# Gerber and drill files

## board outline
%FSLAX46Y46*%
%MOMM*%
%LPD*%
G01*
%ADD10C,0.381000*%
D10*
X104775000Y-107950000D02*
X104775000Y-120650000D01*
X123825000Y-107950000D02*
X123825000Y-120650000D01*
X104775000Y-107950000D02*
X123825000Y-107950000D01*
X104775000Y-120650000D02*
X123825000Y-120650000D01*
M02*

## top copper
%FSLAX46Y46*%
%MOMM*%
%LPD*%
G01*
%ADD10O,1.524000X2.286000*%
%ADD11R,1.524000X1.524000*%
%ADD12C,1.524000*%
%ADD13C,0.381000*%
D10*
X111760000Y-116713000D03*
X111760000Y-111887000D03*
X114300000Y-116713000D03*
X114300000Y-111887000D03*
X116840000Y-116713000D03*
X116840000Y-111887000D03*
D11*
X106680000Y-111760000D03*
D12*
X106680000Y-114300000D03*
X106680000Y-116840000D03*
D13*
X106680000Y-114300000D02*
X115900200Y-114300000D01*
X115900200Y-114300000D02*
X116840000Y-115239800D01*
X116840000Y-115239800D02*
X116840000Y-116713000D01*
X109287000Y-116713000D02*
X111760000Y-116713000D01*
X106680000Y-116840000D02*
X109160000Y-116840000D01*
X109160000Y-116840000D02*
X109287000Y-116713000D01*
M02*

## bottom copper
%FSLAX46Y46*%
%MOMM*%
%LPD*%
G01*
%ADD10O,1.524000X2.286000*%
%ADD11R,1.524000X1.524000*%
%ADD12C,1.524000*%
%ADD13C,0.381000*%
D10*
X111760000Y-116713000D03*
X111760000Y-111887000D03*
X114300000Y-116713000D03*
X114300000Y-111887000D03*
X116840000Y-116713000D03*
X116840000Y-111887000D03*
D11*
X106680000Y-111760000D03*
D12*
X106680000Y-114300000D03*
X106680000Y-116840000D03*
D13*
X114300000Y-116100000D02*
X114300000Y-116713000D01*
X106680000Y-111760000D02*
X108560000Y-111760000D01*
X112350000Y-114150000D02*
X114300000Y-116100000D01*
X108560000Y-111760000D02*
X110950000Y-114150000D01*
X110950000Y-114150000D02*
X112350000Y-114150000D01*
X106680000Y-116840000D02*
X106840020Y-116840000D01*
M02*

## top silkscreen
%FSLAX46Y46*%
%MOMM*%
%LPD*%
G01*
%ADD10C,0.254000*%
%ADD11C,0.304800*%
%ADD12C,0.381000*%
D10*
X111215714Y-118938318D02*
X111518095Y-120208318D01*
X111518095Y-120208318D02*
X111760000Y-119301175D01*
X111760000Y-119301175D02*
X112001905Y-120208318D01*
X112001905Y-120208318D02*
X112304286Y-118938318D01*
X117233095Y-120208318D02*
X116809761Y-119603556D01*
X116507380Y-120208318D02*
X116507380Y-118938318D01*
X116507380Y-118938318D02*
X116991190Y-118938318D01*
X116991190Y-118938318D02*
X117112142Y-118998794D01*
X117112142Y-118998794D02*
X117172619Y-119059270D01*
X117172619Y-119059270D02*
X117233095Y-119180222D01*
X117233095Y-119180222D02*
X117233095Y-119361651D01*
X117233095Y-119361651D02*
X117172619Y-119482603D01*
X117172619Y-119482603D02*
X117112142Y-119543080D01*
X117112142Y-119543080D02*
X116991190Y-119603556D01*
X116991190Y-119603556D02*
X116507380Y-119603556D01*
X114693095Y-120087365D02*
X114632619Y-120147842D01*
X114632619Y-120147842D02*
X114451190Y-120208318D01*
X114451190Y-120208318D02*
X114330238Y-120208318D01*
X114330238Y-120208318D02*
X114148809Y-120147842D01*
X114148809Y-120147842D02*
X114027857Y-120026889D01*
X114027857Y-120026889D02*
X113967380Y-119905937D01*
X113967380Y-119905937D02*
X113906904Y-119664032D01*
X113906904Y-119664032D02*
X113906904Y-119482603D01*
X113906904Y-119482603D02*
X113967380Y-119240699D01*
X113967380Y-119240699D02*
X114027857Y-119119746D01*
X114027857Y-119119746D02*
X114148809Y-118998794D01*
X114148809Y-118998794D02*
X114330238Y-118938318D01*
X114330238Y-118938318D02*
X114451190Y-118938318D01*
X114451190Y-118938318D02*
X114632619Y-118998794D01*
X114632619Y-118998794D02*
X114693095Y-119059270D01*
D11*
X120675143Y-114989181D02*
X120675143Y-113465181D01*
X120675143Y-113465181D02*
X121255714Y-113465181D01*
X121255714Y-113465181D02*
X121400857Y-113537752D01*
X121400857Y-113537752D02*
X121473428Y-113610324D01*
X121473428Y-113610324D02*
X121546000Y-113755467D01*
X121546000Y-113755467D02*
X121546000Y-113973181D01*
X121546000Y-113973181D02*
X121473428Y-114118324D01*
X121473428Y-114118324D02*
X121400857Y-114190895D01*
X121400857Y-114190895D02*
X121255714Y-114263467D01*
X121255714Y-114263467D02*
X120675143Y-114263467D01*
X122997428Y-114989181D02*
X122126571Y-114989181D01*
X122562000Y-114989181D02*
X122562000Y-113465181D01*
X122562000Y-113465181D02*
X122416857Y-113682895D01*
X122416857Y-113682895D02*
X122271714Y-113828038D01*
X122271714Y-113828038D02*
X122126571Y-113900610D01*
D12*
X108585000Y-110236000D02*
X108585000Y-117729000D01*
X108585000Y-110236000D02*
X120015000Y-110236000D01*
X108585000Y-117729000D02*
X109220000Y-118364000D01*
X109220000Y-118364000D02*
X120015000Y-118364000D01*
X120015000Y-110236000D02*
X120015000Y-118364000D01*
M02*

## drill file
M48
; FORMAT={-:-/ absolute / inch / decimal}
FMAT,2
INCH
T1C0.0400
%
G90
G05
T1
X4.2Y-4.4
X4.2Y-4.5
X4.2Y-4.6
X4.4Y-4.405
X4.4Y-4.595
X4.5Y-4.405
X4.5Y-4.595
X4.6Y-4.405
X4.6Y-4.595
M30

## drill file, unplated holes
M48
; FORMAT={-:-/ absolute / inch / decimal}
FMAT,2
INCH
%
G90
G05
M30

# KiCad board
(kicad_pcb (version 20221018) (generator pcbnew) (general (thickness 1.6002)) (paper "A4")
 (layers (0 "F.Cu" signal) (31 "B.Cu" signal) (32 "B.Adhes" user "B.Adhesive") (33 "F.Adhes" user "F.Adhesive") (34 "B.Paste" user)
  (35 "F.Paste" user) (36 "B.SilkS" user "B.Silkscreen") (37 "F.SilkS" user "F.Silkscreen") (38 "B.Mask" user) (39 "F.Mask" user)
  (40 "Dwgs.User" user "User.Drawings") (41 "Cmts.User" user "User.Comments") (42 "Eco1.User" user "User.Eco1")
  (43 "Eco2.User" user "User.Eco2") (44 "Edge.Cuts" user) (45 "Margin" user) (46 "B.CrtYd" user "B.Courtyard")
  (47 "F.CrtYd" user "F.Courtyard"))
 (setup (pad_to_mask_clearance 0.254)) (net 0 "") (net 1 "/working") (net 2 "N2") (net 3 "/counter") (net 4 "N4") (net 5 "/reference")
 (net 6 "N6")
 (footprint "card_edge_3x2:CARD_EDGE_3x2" (layer "F.Cu") (at 114.3 114.3)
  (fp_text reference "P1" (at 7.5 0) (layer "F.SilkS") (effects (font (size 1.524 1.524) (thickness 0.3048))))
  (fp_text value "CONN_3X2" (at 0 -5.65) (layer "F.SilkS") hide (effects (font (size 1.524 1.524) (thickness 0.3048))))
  (fp_line (start -5.715 -4.064) (end -5.715 3.429) (stroke (width 0.381) (type solid)) (layer "F.SilkS"))
  (fp_line (start -5.715 -4.064) (end 5.715 -4.064) (stroke (width 0.381) (type solid)) (layer "F.SilkS"))
  (fp_line (start -5.715 3.429) (end -5.08 4.064) (stroke (width 0.381) (type solid)) (layer "F.SilkS"))
  (fp_line (start -5.08 4.064) (end 5.715 4.064) (stroke (width 0.381) (type solid)) (layer "F.SilkS"))
  (fp_line (start 5.715 -4.064) (end 5.715 4.064) (stroke (width 0.381) (type solid)) (layer "F.SilkS"))
  (pad "1" thru_hole oval (at -2.54 2.413) (size 1.524 2.286) (drill 1.016) (layers "*.Cu" "*.Mask") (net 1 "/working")
   (thermal_bridge_angle 45))
  (pad "2" thru_hole oval (at -2.54 -2.413) (size 1.524 2.286) (drill 1.016) (layers "*.Cu" "*.Mask") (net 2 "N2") (thermal_bridge_angle 45))
  (pad "3" thru_hole oval (at 0 2.413) (size 1.524 2.286) (drill 1.016) (layers "*.Cu" "*.Mask") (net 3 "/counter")
   (thermal_bridge_angle 45))
  (pad "4" thru_hole oval (at 0 -2.413) (size 1.524 2.286) (drill 1.016) (layers "*.Cu" "*.Mask") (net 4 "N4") (thermal_bridge_angle 45))
  (pad "5" thru_hole oval (at 2.54 2.413) (size 1.524 2.286) (drill 1.016) (layers "*.Cu" "*.Mask") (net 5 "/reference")
   (thermal_bridge_angle 45))
  (pad "6" thru_hole oval (at 2.54 -2.413) (size 1.524 2.286) (drill 1.016) (layers "*.Cu" "*.Mask") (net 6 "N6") (thermal_bridge_angle 45)))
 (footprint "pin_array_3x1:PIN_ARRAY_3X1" (layer "B.Cu") (at 106.68 114.3 -90)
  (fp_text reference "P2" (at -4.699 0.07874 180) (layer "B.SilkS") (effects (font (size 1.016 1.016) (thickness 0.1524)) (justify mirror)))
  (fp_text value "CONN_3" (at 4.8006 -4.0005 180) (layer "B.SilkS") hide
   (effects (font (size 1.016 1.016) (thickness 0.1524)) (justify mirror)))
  (pad "1" thru_hole rect (at -2.54 0 270) (size 1.524 1.524) (drill 1.016) (layers "*.Cu" "*.Mask") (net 3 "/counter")
   (thermal_bridge_angle 45))
  (pad "2" thru_hole circle (at 0 0 270) (size 1.524 1.524) (drill 1.016) (layers "*.Cu" "*.Mask") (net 5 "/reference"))
  (pad "3" thru_hole circle (at 2.54 0 270) (size 1.524 1.524) (drill 1.016) (layers "*.Cu" "*.Mask") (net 1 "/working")))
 (gr_line (start 104.775 107.95) (end 104.775 120.65) (stroke (width 0.381) (type solid)) (layer "Edge.Cuts"))
 (gr_line (start 123.825 107.95) (end 123.825 120.65) (stroke (width 0.381) (type solid)) (layer "Edge.Cuts"))
 (gr_line (start 104.775 107.95) (end 123.825 107.95) (stroke (width 0.381) (type solid)) (layer "Edge.Cuts"))
 (gr_line (start 104.775 120.65) (end 123.825 120.65) (stroke (width 0.381) (type solid)) (layer "Edge.Cuts"))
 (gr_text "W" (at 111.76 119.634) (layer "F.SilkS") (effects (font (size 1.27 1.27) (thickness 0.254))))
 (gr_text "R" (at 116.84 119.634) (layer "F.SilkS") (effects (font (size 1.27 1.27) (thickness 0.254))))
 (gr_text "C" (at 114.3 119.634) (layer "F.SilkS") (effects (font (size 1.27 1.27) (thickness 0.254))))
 (segment (start 114.3 116.1) (end 114.3 116.713) (width 0.381) (layer "B.Cu") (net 3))
 (segment (start 106.68 111.76) (end 108.56 111.76) (width 0.381) (layer "B.Cu") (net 3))
 (segment (start 112.35 114.15) (end 114.3 116.1) (width 0.381) (layer "B.Cu") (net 3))
 (segment (start 108.56 111.76) (end 110.95 114.15) (width 0.381) (layer "B.Cu") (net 3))
 (segment (start 110.95 114.15) (end 112.35 114.15) (width 0.381) (layer "B.Cu") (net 3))
 (segment (start 106.68 114.3) (end 115.9002 114.3) (width 0.381) (layer "F.Cu") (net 5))
 (segment (start 115.9002 114.3) (end 116.84 115.2398) (width 0.381) (layer "F.Cu") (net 5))
 (segment (start 116.84 115.2398) (end 116.84 116.713) (width 0.381) (layer "F.Cu") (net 5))
 (segment (start 109.287 116.713) (end 111.76 116.713) (width 0.381) (layer "F.Cu") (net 1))
 (segment (start 106.68 116.84) (end 109.16 116.84) (width 0.381) (layer "F.Cu") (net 1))
 (segment (start 109.16 116.84) (end 109.287 116.713) (width 0.381) (layer "F.Cu") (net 1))
 (segment (start 106.68 116.84) (end 106.84002 116.84) (width 0.381) (layer "B.Cu") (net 1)))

